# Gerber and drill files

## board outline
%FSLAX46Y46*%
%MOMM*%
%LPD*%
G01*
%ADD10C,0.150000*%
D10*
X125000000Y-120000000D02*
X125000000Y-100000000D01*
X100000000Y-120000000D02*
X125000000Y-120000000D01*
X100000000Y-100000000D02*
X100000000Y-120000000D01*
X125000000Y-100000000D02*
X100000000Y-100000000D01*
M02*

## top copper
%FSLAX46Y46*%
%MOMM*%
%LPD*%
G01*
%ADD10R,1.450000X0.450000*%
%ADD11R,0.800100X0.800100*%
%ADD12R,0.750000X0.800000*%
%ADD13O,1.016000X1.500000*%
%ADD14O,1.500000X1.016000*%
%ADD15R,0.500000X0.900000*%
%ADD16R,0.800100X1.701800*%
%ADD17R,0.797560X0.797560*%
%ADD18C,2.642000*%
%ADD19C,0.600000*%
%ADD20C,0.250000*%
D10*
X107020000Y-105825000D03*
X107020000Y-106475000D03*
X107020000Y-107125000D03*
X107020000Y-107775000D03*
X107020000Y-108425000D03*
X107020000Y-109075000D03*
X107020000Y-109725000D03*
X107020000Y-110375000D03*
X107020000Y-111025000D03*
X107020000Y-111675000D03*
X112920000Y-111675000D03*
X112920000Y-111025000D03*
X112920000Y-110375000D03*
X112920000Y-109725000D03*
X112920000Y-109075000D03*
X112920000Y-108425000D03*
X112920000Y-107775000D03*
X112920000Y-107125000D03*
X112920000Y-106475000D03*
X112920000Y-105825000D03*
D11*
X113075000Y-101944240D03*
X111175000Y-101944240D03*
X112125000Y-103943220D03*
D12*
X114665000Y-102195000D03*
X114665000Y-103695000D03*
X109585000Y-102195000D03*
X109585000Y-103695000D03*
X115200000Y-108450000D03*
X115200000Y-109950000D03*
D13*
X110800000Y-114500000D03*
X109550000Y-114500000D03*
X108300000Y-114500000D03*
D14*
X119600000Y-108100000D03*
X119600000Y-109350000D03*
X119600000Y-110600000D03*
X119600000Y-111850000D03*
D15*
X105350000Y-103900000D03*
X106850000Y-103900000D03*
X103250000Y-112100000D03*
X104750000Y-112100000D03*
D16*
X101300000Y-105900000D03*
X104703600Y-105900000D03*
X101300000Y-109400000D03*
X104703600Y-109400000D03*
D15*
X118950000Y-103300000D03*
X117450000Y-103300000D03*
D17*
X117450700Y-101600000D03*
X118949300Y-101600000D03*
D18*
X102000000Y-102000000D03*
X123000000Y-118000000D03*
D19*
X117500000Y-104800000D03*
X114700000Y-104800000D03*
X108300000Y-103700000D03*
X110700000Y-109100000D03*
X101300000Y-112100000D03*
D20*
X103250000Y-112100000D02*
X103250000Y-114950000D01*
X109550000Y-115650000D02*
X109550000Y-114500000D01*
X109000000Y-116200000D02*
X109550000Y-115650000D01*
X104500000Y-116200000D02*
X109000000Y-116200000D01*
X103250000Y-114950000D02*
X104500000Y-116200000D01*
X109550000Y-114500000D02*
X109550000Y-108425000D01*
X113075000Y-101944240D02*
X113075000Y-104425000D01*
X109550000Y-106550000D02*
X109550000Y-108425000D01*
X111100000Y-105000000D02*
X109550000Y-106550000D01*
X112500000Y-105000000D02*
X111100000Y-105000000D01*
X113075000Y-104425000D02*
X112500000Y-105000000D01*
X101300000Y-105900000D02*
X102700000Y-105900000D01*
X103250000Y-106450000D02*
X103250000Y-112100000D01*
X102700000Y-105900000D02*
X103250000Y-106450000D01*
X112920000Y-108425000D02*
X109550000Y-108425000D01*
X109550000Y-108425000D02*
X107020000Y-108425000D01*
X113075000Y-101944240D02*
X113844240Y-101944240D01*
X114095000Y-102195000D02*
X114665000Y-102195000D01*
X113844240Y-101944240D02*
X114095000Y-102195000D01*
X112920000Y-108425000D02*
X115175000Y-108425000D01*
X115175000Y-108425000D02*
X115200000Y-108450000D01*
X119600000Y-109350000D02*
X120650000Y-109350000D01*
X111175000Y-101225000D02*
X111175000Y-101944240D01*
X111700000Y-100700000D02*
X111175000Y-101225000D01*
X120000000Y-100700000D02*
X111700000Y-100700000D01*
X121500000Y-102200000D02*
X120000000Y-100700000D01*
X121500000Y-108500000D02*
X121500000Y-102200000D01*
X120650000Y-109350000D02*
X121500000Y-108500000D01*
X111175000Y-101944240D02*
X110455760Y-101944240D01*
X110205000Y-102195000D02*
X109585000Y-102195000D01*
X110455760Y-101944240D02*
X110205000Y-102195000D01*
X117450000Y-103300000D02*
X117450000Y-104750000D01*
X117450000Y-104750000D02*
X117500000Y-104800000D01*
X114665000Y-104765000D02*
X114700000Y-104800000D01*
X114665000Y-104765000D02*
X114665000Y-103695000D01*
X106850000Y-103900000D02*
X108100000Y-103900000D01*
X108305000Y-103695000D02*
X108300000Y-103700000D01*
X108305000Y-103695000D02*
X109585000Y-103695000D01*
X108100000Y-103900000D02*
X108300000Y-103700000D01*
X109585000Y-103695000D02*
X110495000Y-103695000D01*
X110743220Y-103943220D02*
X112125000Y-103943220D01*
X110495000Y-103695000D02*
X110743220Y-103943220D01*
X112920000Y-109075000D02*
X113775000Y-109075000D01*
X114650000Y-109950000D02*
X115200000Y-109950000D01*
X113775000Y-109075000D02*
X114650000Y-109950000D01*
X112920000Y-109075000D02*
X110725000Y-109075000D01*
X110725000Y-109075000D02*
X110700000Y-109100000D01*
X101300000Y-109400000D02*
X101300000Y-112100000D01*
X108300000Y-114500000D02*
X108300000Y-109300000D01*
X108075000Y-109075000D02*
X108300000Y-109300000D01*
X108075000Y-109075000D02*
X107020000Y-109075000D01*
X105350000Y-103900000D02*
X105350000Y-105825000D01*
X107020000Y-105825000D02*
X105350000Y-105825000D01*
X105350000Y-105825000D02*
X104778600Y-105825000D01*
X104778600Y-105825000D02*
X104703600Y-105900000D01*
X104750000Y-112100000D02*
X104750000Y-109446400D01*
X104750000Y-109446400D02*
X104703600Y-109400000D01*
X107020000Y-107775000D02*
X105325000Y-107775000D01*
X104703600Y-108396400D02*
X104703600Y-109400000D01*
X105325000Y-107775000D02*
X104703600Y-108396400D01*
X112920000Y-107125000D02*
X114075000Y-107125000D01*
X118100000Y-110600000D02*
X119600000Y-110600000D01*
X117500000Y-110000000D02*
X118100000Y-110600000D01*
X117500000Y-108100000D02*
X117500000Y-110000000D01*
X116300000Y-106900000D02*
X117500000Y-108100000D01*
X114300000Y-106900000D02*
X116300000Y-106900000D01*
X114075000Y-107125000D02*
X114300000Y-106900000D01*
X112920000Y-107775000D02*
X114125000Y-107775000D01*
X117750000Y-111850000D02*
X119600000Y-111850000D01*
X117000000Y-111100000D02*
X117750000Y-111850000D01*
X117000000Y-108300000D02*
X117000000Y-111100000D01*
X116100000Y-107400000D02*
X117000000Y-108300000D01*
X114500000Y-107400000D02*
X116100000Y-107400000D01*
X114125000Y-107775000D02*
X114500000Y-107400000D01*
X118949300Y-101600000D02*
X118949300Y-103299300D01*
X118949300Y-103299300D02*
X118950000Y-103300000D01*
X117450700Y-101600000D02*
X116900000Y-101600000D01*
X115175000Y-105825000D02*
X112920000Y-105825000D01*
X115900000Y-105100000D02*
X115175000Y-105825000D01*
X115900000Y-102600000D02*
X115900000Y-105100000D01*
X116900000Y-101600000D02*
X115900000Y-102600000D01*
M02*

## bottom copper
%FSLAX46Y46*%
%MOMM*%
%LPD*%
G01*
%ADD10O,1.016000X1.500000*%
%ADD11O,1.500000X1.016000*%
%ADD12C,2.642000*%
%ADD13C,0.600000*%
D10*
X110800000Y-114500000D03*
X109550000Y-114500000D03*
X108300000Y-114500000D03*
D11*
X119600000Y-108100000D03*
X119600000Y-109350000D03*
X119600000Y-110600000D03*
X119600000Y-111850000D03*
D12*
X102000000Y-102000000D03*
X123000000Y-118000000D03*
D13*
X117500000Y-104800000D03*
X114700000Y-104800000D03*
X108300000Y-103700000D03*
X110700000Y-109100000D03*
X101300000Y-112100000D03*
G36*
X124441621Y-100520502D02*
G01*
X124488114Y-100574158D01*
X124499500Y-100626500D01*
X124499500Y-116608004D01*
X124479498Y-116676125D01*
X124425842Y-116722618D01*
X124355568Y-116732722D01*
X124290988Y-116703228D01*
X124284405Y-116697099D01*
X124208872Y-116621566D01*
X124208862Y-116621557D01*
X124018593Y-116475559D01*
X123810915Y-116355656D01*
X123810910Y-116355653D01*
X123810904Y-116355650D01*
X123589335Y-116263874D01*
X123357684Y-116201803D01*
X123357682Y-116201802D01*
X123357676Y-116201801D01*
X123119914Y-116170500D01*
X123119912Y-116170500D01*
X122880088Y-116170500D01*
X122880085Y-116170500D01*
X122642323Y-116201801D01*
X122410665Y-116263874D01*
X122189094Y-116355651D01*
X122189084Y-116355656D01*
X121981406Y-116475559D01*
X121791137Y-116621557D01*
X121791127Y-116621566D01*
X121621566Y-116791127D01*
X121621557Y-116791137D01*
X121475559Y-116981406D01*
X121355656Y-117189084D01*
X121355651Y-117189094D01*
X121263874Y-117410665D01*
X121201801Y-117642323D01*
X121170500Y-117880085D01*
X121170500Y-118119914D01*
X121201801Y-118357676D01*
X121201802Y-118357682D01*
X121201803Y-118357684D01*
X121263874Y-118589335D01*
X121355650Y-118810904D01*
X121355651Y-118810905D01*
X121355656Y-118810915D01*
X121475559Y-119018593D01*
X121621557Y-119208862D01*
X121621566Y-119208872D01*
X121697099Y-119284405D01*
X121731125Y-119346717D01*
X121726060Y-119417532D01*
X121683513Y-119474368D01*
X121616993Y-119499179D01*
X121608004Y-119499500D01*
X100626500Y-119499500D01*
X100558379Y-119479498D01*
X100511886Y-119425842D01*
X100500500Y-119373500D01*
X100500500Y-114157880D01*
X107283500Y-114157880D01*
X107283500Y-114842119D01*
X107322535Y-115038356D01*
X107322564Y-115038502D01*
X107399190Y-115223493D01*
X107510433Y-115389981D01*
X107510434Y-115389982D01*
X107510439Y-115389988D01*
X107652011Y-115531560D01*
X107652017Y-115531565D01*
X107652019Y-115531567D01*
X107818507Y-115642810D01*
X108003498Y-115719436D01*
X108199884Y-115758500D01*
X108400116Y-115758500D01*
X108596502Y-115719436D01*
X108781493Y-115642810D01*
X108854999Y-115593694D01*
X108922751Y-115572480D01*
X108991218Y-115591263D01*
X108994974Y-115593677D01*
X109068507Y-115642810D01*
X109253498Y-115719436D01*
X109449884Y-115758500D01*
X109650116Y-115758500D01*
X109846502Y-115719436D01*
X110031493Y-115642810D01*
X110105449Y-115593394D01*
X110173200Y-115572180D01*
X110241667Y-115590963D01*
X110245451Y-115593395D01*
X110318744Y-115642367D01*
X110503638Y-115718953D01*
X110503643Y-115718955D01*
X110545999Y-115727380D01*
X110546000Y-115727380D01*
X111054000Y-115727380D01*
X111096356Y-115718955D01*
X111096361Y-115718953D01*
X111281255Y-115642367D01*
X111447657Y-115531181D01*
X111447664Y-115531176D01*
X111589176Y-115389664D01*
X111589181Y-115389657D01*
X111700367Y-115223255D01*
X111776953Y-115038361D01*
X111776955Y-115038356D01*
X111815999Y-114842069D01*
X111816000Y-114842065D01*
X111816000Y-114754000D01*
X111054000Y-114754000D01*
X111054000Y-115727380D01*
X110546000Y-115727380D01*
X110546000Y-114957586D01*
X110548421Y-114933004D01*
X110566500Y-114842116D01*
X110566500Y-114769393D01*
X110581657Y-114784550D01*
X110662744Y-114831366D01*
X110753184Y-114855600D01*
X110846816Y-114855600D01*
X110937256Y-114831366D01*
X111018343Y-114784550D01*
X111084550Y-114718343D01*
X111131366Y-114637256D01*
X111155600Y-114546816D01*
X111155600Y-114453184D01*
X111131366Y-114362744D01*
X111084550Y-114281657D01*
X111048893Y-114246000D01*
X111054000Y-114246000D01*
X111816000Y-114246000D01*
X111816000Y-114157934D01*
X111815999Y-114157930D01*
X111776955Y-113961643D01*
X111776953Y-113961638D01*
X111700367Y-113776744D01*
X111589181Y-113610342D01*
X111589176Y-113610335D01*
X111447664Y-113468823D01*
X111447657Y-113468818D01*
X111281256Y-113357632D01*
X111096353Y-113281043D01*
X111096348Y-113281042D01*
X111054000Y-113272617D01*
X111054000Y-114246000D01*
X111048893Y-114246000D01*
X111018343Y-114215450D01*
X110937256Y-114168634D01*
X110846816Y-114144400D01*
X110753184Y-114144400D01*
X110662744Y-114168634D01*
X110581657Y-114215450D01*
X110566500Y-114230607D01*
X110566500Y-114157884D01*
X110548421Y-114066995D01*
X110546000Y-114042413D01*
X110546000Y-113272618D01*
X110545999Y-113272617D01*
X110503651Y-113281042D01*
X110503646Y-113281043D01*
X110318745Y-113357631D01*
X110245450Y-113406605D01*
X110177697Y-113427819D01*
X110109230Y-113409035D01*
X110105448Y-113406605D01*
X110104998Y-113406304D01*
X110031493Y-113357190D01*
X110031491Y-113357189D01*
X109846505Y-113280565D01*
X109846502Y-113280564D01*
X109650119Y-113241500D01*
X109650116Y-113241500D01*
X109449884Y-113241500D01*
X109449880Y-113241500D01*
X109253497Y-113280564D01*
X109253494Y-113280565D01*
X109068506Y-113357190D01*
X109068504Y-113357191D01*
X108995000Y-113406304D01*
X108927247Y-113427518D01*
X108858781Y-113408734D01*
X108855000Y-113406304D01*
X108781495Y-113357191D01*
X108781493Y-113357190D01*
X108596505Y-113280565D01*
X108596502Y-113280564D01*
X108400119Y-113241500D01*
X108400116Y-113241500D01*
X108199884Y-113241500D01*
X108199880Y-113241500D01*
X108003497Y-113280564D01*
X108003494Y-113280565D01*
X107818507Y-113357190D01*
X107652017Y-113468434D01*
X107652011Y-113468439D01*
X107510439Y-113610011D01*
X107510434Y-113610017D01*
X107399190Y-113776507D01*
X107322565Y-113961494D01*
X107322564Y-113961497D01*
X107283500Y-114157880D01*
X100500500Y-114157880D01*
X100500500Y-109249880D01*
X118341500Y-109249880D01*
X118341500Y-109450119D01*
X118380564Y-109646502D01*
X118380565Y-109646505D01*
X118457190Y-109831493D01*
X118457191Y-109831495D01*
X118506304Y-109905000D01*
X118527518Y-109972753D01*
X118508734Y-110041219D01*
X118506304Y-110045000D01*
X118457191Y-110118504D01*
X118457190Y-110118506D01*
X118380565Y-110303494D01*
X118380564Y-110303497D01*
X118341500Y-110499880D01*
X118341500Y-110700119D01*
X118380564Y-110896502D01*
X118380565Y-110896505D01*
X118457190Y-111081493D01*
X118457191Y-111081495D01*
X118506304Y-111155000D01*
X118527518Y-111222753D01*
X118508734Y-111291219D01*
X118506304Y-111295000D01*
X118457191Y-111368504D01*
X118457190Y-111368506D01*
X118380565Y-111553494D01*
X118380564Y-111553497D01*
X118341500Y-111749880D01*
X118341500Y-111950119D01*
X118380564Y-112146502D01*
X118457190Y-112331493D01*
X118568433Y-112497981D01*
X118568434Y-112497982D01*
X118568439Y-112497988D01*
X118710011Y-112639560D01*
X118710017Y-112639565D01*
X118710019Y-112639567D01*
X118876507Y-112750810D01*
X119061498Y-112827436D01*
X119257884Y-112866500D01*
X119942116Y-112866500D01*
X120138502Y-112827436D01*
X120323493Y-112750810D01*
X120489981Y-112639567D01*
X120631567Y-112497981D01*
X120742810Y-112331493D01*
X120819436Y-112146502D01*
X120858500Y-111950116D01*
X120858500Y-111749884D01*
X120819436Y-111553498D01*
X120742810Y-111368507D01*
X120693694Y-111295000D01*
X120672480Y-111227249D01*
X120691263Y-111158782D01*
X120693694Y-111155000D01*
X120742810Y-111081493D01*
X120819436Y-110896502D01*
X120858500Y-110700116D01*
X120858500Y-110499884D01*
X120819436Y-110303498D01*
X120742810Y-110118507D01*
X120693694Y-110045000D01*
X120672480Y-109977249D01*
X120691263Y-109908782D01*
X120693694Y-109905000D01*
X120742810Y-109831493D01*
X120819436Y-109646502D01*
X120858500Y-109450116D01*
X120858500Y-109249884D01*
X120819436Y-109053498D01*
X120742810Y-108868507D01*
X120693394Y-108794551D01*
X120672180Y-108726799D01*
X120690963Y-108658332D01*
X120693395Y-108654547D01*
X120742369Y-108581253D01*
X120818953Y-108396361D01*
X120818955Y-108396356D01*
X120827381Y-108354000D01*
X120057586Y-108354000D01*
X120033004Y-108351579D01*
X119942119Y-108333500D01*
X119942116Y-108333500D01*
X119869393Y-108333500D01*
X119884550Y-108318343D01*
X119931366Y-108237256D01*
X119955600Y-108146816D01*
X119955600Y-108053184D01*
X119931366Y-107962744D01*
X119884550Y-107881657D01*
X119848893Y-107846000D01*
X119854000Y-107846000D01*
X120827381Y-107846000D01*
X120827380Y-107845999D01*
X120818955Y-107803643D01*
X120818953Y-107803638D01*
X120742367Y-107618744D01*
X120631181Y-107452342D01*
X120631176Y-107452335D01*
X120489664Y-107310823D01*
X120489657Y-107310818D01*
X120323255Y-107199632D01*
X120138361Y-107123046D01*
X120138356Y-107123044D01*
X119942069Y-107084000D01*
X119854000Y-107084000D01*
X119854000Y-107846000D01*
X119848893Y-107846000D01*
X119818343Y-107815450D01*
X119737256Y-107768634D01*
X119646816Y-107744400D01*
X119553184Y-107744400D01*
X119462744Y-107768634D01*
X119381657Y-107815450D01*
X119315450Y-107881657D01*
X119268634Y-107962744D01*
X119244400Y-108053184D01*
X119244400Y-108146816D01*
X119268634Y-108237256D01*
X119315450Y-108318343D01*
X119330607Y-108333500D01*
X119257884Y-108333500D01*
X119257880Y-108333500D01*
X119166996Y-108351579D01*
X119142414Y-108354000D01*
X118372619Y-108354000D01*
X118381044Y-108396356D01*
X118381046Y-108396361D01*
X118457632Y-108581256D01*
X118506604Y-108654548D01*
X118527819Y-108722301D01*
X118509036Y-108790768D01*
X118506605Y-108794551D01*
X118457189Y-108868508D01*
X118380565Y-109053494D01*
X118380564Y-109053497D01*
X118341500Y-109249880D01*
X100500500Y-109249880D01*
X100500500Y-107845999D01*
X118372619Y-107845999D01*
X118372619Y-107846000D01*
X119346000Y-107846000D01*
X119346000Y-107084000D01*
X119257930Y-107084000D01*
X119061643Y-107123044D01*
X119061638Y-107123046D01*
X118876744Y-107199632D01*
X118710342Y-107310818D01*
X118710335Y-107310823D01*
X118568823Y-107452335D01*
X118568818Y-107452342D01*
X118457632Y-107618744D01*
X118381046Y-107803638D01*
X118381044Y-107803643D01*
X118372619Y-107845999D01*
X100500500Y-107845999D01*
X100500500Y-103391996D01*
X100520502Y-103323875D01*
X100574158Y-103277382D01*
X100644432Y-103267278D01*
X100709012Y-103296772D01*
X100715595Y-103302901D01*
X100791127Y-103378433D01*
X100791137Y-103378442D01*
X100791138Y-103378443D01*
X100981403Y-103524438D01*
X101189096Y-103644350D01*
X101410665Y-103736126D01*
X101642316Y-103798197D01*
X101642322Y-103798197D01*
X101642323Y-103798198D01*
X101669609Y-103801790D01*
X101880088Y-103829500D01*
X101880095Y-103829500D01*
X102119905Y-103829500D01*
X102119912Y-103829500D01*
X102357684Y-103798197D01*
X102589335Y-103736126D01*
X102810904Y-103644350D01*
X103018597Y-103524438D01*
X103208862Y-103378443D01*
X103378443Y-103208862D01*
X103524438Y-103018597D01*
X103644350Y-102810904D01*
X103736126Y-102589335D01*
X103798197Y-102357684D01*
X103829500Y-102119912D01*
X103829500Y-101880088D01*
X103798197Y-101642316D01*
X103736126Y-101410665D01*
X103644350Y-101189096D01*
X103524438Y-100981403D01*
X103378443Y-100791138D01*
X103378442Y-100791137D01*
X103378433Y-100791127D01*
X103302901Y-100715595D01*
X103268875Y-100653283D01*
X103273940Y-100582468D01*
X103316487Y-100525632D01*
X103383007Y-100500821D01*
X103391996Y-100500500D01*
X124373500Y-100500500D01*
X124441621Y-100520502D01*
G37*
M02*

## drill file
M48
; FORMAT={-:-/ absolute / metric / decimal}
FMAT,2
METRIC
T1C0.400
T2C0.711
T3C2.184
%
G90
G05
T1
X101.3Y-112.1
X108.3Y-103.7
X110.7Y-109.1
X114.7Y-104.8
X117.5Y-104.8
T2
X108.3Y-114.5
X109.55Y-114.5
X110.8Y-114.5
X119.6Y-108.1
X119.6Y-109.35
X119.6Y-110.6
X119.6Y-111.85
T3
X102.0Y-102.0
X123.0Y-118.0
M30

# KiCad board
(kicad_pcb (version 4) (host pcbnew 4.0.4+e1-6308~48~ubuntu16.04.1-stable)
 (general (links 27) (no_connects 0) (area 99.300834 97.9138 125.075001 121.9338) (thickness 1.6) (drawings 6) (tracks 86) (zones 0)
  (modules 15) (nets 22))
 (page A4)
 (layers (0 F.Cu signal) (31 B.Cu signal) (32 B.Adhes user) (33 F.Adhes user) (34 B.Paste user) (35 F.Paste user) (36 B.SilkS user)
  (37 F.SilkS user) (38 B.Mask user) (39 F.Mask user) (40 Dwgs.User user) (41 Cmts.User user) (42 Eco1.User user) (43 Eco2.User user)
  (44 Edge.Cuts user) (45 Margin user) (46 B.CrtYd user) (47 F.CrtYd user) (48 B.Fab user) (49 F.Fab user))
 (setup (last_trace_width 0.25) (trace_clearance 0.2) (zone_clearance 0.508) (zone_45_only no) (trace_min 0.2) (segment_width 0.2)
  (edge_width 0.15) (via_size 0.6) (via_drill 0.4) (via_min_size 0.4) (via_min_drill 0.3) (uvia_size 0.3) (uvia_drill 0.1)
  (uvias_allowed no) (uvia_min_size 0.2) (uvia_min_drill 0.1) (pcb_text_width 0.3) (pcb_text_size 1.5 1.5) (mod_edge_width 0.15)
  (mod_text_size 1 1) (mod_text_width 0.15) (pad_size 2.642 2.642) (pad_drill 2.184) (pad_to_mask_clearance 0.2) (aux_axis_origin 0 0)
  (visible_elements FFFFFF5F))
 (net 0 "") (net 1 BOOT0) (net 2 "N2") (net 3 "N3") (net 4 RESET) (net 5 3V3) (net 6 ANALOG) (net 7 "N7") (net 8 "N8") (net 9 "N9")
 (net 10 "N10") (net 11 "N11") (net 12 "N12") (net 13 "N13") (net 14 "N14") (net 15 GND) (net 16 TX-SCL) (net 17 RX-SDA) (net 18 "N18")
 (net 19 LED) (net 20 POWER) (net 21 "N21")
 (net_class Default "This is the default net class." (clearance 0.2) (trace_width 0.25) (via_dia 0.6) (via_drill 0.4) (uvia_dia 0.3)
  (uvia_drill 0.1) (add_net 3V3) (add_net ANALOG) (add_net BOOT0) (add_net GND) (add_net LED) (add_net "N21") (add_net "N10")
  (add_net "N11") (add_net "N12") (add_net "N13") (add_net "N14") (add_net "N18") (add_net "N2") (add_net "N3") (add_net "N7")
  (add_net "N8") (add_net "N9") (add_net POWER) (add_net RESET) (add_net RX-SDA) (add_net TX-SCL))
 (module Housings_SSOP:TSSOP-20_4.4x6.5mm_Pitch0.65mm (layer F.Cu) (at 109.97 108.75)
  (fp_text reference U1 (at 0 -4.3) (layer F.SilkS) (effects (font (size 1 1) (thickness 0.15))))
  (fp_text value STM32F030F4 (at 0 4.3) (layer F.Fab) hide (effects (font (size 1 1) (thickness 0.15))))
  (pad 1 smd rect (at -2.95 -2.925) (size 1.45 0.45) (layers F.Cu F.Paste F.Mask) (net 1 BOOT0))
  (pad 2 smd rect (at -2.95 -2.275) (size 1.45 0.45) (layers F.Cu F.Paste F.Mask) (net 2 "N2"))
  (pad 3 smd rect (at -2.95 -1.625) (size 1.45 0.45) (layers F.Cu F.Paste F.Mask) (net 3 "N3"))
  (pad 4 smd rect (at -2.95 -0.975) (size 1.45 0.45) (layers F.Cu F.Paste F.Mask) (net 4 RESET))
  (pad 5 smd rect (at -2.95 -0.325) (size 1.45 0.45) (layers F.Cu F.Paste F.Mask) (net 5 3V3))
  (pad 6 smd rect (at -2.95 0.325) (size 1.45 0.45) (layers F.Cu F.Paste F.Mask) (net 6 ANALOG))
  (pad 7 smd rect (at -2.95 0.975) (size 1.45 0.45) (layers F.Cu F.Paste F.Mask) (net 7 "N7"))
  (pad 8 smd rect (at -2.95 1.625) (size 1.45 0.45) (layers F.Cu F.Paste F.Mask) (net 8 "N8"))
  (pad 9 smd rect (at -2.95 2.275) (size 1.45 0.45) (layers F.Cu F.Paste F.Mask) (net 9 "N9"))
  (pad 10 smd rect (at -2.95 2.925) (size 1.45 0.45) (layers F.Cu F.Paste F.Mask) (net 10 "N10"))
  (pad 11 smd rect (at 2.95 2.925) (size 1.45 0.45) (layers F.Cu F.Paste F.Mask) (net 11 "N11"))
  (pad 12 smd rect (at 2.95 2.275) (size 1.45 0.45) (layers F.Cu F.Paste F.Mask) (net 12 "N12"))
  (pad 13 smd rect (at 2.95 1.625) (size 1.45 0.45) (layers F.Cu F.Paste F.Mask) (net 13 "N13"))
  (pad 14 smd rect (at 2.95 0.975) (size 1.45 0.45) (layers F.Cu F.Paste F.Mask) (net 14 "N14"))
  (pad 15 smd rect (at 2.95 0.325) (size 1.45 0.45) (layers F.Cu F.Paste F.Mask) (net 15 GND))
  (pad 16 smd rect (at 2.95 -0.325) (size 1.45 0.45) (layers F.Cu F.Paste F.Mask) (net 5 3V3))
  (pad 17 smd rect (at 2.95 -0.975) (size 1.45 0.45) (layers F.Cu F.Paste F.Mask) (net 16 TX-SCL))
  (pad 18 smd rect (at 2.95 -1.625) (size 1.45 0.45) (layers F.Cu F.Paste F.Mask) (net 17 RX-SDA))
  (pad 19 smd rect (at 2.95 -2.275) (size 1.45 0.45) (layers F.Cu F.Paste F.Mask) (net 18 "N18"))
  (pad 20 smd rect (at 2.95 -2.925) (size 1.45 0.45) (layers F.Cu F.Paste F.Mask) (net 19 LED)))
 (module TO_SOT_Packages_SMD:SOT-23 (layer F.Cu) (at 112.125 102.945 180)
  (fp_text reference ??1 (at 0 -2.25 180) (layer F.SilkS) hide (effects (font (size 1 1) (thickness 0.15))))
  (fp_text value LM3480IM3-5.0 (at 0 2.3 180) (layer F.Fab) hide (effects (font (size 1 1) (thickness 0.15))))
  (pad 1 smd rect (at -0.95 1.00076 180) (size 0.8001 0.8001) (layers F.Cu F.Paste F.Mask) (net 5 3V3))
  (pad 2 smd rect (at 0.95 1.00076 180) (size 0.8001 0.8001) (layers F.Cu F.Paste F.Mask) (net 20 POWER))
  (pad 3 smd rect (at 0 -0.99822 180) (size 0.8001 0.8001) (layers F.Cu F.Paste F.Mask) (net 15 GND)))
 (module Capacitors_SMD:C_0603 (layer F.Cu) (at 114.665 102.945 270)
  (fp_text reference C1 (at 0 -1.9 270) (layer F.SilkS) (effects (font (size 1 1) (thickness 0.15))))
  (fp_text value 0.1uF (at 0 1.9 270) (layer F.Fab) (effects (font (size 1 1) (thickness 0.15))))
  (pad 1 smd rect (at -0.75 0 270) (size 0.8 0.75) (layers F.Cu F.Paste F.Mask) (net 5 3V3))
  (pad 2 smd rect (at 0.75 0 270) (size 0.8 0.75) (layers F.Cu F.Paste F.Mask) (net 15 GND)))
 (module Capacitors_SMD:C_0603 (layer F.Cu) (at 109.585 102.945 270)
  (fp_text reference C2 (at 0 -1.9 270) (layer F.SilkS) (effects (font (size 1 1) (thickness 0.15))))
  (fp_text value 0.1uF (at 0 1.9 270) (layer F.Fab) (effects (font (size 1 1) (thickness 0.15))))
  (pad 1 smd rect (at -0.75 0 270) (size 0.8 0.75) (layers F.Cu F.Paste F.Mask) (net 20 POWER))
  (pad 2 smd rect (at 0.75 0 270) (size 0.8 0.75) (layers F.Cu F.Paste F.Mask) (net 15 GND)))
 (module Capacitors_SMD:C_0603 (layer F.Cu) (at 115.2 109.2 270)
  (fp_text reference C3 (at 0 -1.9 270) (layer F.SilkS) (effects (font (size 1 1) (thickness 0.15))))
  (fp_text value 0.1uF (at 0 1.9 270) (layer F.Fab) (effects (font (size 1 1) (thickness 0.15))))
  (pad 1 smd rect (at -0.75 0 270) (size 0.8 0.75) (layers F.Cu F.Paste F.Mask) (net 5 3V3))
  (pad 2 smd rect (at 0.75 0 270) (size 0.8 0.75) (layers F.Cu F.Paste F.Mask) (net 15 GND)))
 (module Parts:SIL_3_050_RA (layer F.Cu) (at 110.8 114.5 180)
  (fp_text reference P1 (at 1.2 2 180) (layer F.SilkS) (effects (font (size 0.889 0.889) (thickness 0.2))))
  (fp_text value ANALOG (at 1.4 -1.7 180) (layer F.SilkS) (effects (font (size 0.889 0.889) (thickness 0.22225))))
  (pad 1 thru_hole oval (at 0 0 180) (size 1.016 1.5) (drill 0.7112) (layers *.Cu *.Mask F.SilkS) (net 15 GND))
  (pad 2 thru_hole oval (at 1.25 0 180) (size 1.016 1.5) (drill 0.7112) (layers *.Cu *.Mask F.SilkS) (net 5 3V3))
  (pad 3 thru_hole oval (at 2.5 0 180) (size 1.016 1.5) (drill 0.7112) (layers *.Cu *.Mask F.SilkS) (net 6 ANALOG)))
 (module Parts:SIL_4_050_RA (layer F.Cu) (at 119.6 108.1 270)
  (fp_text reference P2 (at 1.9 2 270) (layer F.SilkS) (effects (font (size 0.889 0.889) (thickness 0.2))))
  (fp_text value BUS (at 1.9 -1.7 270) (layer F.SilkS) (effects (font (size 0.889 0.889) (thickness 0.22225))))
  (pad 1 thru_hole oval (at 0 0 270) (size 1.016 1.5) (drill 0.7112) (layers *.Cu *.Mask F.SilkS) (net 15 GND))
  (pad 2 thru_hole oval (at 1.25 0 270) (size 1.016 1.5) (drill 0.7112) (layers *.Cu *.Mask F.SilkS) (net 20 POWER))
  (pad 3 thru_hole oval (at 2.5 0 270) (size 1.016 1.5) (drill 0.7112) (layers *.Cu *.Mask F.SilkS) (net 17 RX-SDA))
  (pad 4 thru_hole oval (at 3.75 0 270) (size 1.016 1.5) (drill 0.7112) (layers *.Cu *.Mask F.SilkS) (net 16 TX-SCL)))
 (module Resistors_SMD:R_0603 (layer F.Cu) (at 106.1 103.9)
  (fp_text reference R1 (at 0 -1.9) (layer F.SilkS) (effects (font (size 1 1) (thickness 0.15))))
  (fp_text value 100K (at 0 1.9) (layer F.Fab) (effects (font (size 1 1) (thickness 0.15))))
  (pad 1 smd rect (at -0.75 0) (size 0.5 0.9) (layers F.Cu F.Paste F.Mask) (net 1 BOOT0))
  (pad 2 smd rect (at 0.75 0) (size 0.5 0.9) (layers F.Cu F.Paste F.Mask) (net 15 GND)))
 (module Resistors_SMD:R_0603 (layer F.Cu) (at 104 112.1)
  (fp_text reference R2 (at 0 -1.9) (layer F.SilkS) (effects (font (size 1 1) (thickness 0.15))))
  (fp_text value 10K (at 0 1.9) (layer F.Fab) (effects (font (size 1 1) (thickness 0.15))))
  (pad 1 smd rect (at -0.75 0) (size 0.5 0.9) (layers F.Cu F.Paste F.Mask) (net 5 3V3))
  (pad 2 smd rect (at 0.75 0) (size 0.5 0.9) (layers F.Cu F.Paste F.Mask) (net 4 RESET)))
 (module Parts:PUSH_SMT (layer F.Cu) (at 101.3 105.9)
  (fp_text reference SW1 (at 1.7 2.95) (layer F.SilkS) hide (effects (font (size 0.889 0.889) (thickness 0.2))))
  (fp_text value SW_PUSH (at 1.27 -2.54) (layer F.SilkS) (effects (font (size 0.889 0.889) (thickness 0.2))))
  (pad 1 smd rect (at 0 0) (size 0.8001 1.7018) (layers F.Cu F.Paste F.Mask) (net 5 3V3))
  (pad 2 smd rect (at 3.4036 0) (size 0.8001 1.7018) (layers F.Cu F.Paste F.Mask) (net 1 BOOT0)))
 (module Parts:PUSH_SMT (layer F.Cu) (at 101.3 109.4)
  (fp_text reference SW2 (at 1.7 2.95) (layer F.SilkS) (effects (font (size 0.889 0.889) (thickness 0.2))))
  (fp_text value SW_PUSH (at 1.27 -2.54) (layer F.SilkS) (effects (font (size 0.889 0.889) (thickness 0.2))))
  (pad 1 smd rect (at 0 0) (size 0.8001 1.7018) (layers F.Cu F.Paste F.Mask) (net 15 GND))
  (pad 2 smd rect (at 3.4036 0) (size 0.8001 1.7018) (layers F.Cu F.Paste F.Mask) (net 4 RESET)))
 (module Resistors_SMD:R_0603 (layer F.Cu) (at 118.2 103.3 180)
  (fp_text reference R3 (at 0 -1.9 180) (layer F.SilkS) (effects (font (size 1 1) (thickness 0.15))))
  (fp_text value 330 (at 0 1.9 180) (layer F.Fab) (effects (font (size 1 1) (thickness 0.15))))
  (pad 1 smd rect (at -0.75 0 180) (size 0.5 0.9) (layers F.Cu F.Paste F.Mask) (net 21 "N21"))
  (pad 2 smd rect (at 0.75 0 180) (size 0.5 0.9) (layers F.Cu F.Paste F.Mask) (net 15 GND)))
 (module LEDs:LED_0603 (layer F.Cu) (at 118.2 101.6 180)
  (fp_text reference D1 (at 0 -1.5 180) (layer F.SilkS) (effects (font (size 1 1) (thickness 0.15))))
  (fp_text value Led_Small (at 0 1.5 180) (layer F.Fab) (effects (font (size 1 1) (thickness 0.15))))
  (pad 2 smd rect (at 0.7493 0) (size 0.79756 0.79756) (layers F.Cu F.Paste F.Mask) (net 19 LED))
  (pad 1 smd rect (at -0.7493 0) (size 0.79756 0.79756) (layers F.Cu F.Paste F.Mask) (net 21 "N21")))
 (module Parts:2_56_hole (layer F.Cu) (at 102 102)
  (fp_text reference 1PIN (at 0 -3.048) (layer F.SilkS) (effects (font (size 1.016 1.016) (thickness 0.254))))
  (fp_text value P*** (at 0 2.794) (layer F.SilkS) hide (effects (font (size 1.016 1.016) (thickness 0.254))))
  (pad "" thru_hole circle (at 0 0) (size 2.642 2.642) (drill 2.184) (layers *.Cu *.Mask F.SilkS)))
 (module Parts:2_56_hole (layer F.Cu) (at 123 118)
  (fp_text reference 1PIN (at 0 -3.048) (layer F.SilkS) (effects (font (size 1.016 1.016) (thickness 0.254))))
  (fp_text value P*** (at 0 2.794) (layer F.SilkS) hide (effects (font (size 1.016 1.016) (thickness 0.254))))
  (pad "" thru_hole circle (at 0 0) (size 2.642 2.642) (drill 2.184) (layers *.Cu *.Mask F.SilkS)))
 (gr_line (start 125 120) (end 125 100) (angle 90) (layer Edge.Cuts) (width 0.15))
 (gr_line (start 100 120) (end 125 120) (angle 90) (layer Edge.Cuts) (width 0.15))
 (gr_line (start 100 100) (end 100 120) (angle 90) (layer Edge.Cuts) (width 0.15))
 (gr_line (start 125 100) (end 100 100) (angle 90) (layer Edge.Cuts) (width 0.15))
 (segment (start 103.25 112.1) (end 103.25 114.95) (width 0.25) (layer F.Cu) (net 5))
 (segment (start 109.55 115.65) (end 109.55 114.5) (width 0.25) (layer F.Cu) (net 5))
 (segment (start 109 116.2) (end 109.55 115.65) (width 0.25) (layer F.Cu) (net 5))
 (segment (start 104.5 116.2) (end 109 116.2) (width 0.25) (layer F.Cu) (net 5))
 (segment (start 103.25 114.95) (end 104.5 116.2) (width 0.25) (layer F.Cu) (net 5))
 (segment (start 109.55 114.5) (end 109.55 108.425) (width 0.25) (layer F.Cu) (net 5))
 (segment (start 113.075 101.94424) (end 113.075 104.425) (width 0.25) (layer F.Cu) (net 5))
 (segment (start 109.55 106.55) (end 109.55 108.425) (width 0.25) (layer F.Cu) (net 5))
 (segment (start 111.1 105) (end 109.55 106.55) (width 0.25) (layer F.Cu) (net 5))
 (segment (start 112.5 105) (end 111.1 105) (width 0.25) (layer F.Cu) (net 5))
 (segment (start 113.075 104.425) (end 112.5 105) (width 0.25) (layer F.Cu) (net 5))
 (segment (start 101.3 105.9) (end 102.7 105.9) (width 0.25) (layer F.Cu) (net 5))
 (segment (start 103.25 106.45) (end 103.25 112.1) (width 0.25) (layer F.Cu) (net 5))
 (segment (start 102.7 105.9) (end 103.25 106.45) (width 0.25) (layer F.Cu) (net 5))
 (segment (start 112.92 108.425) (end 109.55 108.425) (width 0.25) (layer F.Cu) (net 5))
 (segment (start 109.55 108.425) (end 107.02 108.425) (width 0.25) (layer F.Cu) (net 5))
 (segment (start 113.075 101.94424) (end 113.84424 101.94424) (width 0.25) (layer F.Cu) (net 5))
 (segment (start 114.095 102.195) (end 114.665 102.195) (width 0.25) (layer F.Cu) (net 5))
 (segment (start 113.84424 101.94424) (end 114.095 102.195) (width 0.25) (layer F.Cu) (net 5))
 (segment (start 112.92 108.425) (end 115.175 108.425) (width 0.25) (layer F.Cu) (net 5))
 (segment (start 115.175 108.425) (end 115.2 108.45) (width 0.25) (layer F.Cu) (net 5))
 (segment (start 119.6 109.35) (end 120.65 109.35) (width 0.25) (layer F.Cu) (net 20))
 (segment (start 111.175 101.225) (end 111.175 101.94424) (width 0.25) (layer F.Cu) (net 20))
 (segment (start 111.7 100.7) (end 111.175 101.225) (width 0.25) (layer F.Cu) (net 20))
 (segment (start 120 100.7) (end 111.7 100.7) (width 0.25) (layer F.Cu) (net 20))
 (segment (start 121.5 102.2) (end 120 100.7) (width 0.25) (layer F.Cu) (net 20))
 (segment (start 121.5 108.5) (end 121.5 102.2) (width 0.25) (layer F.Cu) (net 20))
 (segment (start 120.65 109.35) (end 121.5 108.5) (width 0.25) (layer F.Cu) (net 20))
 (segment (start 111.175 101.94424) (end 110.45576 101.94424) (width 0.25) (layer F.Cu) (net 20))
 (segment (start 110.205 102.195) (end 109.585 102.195) (width 0.25) (layer F.Cu) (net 20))
 (segment (start 110.45576 101.94424) (end 110.205 102.195) (width 0.25) (layer F.Cu) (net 20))
 (segment (start 117.45 103.3) (end 117.45 104.75) (width 0.25) (layer F.Cu) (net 15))
 (via (at 117.5 104.8) (size 0.6) (drill 0.4) (layers F.Cu B.Cu) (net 15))
 (segment (start 117.45 104.75) (end 117.5 104.8) (width 0.25) (layer F.Cu) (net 15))
 (segment (start 114.665 104.765) (end 114.7 104.8) (width 0.25) (layer F.Cu) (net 15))
 (via (at 114.7 104.8) (size 0.6) (drill 0.4) (layers F.Cu B.Cu) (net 15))
 (segment (start 114.665 104.765) (end 114.665 103.695) (width 0.25) (layer F.Cu) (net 15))
 (segment (start 106.85 103.9) (end 108.1 103.9) (width 0.25) (layer F.Cu) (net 15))
 (segment (start 108.305 103.695) (end 108.3 103.7) (width 0.25) (layer F.Cu) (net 15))
 (via (at 108.3 103.7) (size 0.6) (drill 0.4) (layers F.Cu B.Cu) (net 15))
 (segment (start 108.305 103.695) (end 109.585 103.695) (width 0.25) (layer F.Cu) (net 15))
 (segment (start 108.1 103.9) (end 108.3 103.7) (width 0.25) (layer F.Cu) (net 15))
 (segment (start 109.585 103.695) (end 110.495 103.695) (width 0.25) (layer F.Cu) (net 15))
 (segment (start 110.74322 103.94322) (end 112.125 103.94322) (width 0.25) (layer F.Cu) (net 15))
 (segment (start 110.495 103.695) (end 110.74322 103.94322) (width 0.25) (layer F.Cu) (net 15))
 (segment (start 112.92 109.075) (end 113.775 109.075) (width 0.25) (layer F.Cu) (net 15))
 (segment (start 114.65 109.95) (end 115.2 109.95) (width 0.25) (layer F.Cu) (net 15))
 (segment (start 113.775 109.075) (end 114.65 109.95) (width 0.25) (layer F.Cu) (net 15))
 (segment (start 112.92 109.075) (end 110.725 109.075) (width 0.25) (layer F.Cu) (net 15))
 (via (at 110.7 109.1) (size 0.6) (drill 0.4) (layers F.Cu B.Cu) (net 15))
 (segment (start 110.725 109.075) (end 110.7 109.1) (width 0.25) (layer F.Cu) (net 15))
 (segment (start 101.3 109.4) (end 101.3 112.1) (width 0.25) (layer F.Cu) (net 15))
 (via (at 101.3 112.1) (size 0.6) (drill 0.4) (layers F.Cu B.Cu) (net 15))
 (segment (start 108.3 114.5) (end 108.3 109.3) (width 0.25) (layer F.Cu) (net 6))
 (segment (start 108.075 109.075) (end 108.3 109.3) (width 0.25) (layer F.Cu) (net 6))
 (segment (start 108.075 109.075) (end 107.02 109.075) (width 0.25) (layer F.Cu) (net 6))
 (segment (start 105.35 103.9) (end 105.35 105.825) (width 0.25) (layer F.Cu) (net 1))
 (segment (start 107.02 105.825) (end 105.35 105.825) (width 0.25) (layer F.Cu) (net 1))
 (segment (start 105.35 105.825) (end 104.7786 105.825) (width 0.25) (layer F.Cu) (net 1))
 (segment (start 104.7786 105.825) (end 104.7036 105.9) (width 0.25) (layer F.Cu) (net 1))
 (segment (start 104.75 112.1) (end 104.75 109.4464) (width 0.25) (layer F.Cu) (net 4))
 (segment (start 104.75 109.4464) (end 104.7036 109.4) (width 0.25) (layer F.Cu) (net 4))
 (segment (start 107.02 107.775) (end 105.325 107.775) (width 0.25) (layer F.Cu) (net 4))
 (segment (start 104.7036 108.3964) (end 104.7036 109.4) (width 0.25) (layer F.Cu) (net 4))
 (segment (start 105.325 107.775) (end 104.7036 108.3964) (width 0.25) (layer F.Cu) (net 4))
 (segment (start 112.92 107.125) (end 114.075 107.125) (width 0.25) (layer F.Cu) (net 17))
 (segment (start 118.1 110.6) (end 119.6 110.6) (width 0.25) (layer F.Cu) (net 17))
 (segment (start 117.5 110) (end 118.1 110.6) (width 0.25) (layer F.Cu) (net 17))
 (segment (start 117.5 108.1) (end 117.5 110) (width 0.25) (layer F.Cu) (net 17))
 (segment (start 116.3 106.9) (end 117.5 108.1) (width 0.25) (layer F.Cu) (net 17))
 (segment (start 114.3 106.9) (end 116.3 106.9) (width 0.25) (layer F.Cu) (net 17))
 (segment (start 114.075 107.125) (end 114.3 106.9) (width 0.25) (layer F.Cu) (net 17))
 (segment (start 112.92 107.775) (end 114.125 107.775) (width 0.25) (layer F.Cu) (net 16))
 (segment (start 117.75 111.85) (end 119.6 111.85) (width 0.25) (layer F.Cu) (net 16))
 (segment (start 117 111.1) (end 117.75 111.85) (width 0.25) (layer F.Cu) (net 16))
 (segment (start 117 108.3) (end 117 111.1) (width 0.25) (layer F.Cu) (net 16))
 (segment (start 116.1 107.4) (end 117 108.3) (width 0.25) (layer F.Cu) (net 16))
 (segment (start 114.5 107.4) (end 116.1 107.4) (width 0.25) (layer F.Cu) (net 16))
 (segment (start 114.125 107.775) (end 114.5 107.4) (width 0.25) (layer F.Cu) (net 16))
 (segment (start 118.9493 101.6) (end 118.9493 103.2993) (width 0.25) (layer F.Cu) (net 21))
 (segment (start 118.9493 103.2993) (end 118.95 103.3) (width 0.25) (layer F.Cu) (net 21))
 (segment (start 117.4507 101.6) (end 116.9 101.6) (width 0.25) (layer F.Cu) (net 19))
 (segment (start 115.175 105.825) (end 112.92 105.825) (width 0.25) (layer F.Cu) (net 19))
 (segment (start 115.9 105.1) (end 115.175 105.825) (width 0.25) (layer F.Cu) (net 19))
 (segment (start 115.9 102.6) (end 115.9 105.1) (width 0.25) (layer F.Cu) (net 19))
 (segment (start 116.9 101.6) (end 115.9 102.6) (width 0.25) (layer F.Cu) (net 19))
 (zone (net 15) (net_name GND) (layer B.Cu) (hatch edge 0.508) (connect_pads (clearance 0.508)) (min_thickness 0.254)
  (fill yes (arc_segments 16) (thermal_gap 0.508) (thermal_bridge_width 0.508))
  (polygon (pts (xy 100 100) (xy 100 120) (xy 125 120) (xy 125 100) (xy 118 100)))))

